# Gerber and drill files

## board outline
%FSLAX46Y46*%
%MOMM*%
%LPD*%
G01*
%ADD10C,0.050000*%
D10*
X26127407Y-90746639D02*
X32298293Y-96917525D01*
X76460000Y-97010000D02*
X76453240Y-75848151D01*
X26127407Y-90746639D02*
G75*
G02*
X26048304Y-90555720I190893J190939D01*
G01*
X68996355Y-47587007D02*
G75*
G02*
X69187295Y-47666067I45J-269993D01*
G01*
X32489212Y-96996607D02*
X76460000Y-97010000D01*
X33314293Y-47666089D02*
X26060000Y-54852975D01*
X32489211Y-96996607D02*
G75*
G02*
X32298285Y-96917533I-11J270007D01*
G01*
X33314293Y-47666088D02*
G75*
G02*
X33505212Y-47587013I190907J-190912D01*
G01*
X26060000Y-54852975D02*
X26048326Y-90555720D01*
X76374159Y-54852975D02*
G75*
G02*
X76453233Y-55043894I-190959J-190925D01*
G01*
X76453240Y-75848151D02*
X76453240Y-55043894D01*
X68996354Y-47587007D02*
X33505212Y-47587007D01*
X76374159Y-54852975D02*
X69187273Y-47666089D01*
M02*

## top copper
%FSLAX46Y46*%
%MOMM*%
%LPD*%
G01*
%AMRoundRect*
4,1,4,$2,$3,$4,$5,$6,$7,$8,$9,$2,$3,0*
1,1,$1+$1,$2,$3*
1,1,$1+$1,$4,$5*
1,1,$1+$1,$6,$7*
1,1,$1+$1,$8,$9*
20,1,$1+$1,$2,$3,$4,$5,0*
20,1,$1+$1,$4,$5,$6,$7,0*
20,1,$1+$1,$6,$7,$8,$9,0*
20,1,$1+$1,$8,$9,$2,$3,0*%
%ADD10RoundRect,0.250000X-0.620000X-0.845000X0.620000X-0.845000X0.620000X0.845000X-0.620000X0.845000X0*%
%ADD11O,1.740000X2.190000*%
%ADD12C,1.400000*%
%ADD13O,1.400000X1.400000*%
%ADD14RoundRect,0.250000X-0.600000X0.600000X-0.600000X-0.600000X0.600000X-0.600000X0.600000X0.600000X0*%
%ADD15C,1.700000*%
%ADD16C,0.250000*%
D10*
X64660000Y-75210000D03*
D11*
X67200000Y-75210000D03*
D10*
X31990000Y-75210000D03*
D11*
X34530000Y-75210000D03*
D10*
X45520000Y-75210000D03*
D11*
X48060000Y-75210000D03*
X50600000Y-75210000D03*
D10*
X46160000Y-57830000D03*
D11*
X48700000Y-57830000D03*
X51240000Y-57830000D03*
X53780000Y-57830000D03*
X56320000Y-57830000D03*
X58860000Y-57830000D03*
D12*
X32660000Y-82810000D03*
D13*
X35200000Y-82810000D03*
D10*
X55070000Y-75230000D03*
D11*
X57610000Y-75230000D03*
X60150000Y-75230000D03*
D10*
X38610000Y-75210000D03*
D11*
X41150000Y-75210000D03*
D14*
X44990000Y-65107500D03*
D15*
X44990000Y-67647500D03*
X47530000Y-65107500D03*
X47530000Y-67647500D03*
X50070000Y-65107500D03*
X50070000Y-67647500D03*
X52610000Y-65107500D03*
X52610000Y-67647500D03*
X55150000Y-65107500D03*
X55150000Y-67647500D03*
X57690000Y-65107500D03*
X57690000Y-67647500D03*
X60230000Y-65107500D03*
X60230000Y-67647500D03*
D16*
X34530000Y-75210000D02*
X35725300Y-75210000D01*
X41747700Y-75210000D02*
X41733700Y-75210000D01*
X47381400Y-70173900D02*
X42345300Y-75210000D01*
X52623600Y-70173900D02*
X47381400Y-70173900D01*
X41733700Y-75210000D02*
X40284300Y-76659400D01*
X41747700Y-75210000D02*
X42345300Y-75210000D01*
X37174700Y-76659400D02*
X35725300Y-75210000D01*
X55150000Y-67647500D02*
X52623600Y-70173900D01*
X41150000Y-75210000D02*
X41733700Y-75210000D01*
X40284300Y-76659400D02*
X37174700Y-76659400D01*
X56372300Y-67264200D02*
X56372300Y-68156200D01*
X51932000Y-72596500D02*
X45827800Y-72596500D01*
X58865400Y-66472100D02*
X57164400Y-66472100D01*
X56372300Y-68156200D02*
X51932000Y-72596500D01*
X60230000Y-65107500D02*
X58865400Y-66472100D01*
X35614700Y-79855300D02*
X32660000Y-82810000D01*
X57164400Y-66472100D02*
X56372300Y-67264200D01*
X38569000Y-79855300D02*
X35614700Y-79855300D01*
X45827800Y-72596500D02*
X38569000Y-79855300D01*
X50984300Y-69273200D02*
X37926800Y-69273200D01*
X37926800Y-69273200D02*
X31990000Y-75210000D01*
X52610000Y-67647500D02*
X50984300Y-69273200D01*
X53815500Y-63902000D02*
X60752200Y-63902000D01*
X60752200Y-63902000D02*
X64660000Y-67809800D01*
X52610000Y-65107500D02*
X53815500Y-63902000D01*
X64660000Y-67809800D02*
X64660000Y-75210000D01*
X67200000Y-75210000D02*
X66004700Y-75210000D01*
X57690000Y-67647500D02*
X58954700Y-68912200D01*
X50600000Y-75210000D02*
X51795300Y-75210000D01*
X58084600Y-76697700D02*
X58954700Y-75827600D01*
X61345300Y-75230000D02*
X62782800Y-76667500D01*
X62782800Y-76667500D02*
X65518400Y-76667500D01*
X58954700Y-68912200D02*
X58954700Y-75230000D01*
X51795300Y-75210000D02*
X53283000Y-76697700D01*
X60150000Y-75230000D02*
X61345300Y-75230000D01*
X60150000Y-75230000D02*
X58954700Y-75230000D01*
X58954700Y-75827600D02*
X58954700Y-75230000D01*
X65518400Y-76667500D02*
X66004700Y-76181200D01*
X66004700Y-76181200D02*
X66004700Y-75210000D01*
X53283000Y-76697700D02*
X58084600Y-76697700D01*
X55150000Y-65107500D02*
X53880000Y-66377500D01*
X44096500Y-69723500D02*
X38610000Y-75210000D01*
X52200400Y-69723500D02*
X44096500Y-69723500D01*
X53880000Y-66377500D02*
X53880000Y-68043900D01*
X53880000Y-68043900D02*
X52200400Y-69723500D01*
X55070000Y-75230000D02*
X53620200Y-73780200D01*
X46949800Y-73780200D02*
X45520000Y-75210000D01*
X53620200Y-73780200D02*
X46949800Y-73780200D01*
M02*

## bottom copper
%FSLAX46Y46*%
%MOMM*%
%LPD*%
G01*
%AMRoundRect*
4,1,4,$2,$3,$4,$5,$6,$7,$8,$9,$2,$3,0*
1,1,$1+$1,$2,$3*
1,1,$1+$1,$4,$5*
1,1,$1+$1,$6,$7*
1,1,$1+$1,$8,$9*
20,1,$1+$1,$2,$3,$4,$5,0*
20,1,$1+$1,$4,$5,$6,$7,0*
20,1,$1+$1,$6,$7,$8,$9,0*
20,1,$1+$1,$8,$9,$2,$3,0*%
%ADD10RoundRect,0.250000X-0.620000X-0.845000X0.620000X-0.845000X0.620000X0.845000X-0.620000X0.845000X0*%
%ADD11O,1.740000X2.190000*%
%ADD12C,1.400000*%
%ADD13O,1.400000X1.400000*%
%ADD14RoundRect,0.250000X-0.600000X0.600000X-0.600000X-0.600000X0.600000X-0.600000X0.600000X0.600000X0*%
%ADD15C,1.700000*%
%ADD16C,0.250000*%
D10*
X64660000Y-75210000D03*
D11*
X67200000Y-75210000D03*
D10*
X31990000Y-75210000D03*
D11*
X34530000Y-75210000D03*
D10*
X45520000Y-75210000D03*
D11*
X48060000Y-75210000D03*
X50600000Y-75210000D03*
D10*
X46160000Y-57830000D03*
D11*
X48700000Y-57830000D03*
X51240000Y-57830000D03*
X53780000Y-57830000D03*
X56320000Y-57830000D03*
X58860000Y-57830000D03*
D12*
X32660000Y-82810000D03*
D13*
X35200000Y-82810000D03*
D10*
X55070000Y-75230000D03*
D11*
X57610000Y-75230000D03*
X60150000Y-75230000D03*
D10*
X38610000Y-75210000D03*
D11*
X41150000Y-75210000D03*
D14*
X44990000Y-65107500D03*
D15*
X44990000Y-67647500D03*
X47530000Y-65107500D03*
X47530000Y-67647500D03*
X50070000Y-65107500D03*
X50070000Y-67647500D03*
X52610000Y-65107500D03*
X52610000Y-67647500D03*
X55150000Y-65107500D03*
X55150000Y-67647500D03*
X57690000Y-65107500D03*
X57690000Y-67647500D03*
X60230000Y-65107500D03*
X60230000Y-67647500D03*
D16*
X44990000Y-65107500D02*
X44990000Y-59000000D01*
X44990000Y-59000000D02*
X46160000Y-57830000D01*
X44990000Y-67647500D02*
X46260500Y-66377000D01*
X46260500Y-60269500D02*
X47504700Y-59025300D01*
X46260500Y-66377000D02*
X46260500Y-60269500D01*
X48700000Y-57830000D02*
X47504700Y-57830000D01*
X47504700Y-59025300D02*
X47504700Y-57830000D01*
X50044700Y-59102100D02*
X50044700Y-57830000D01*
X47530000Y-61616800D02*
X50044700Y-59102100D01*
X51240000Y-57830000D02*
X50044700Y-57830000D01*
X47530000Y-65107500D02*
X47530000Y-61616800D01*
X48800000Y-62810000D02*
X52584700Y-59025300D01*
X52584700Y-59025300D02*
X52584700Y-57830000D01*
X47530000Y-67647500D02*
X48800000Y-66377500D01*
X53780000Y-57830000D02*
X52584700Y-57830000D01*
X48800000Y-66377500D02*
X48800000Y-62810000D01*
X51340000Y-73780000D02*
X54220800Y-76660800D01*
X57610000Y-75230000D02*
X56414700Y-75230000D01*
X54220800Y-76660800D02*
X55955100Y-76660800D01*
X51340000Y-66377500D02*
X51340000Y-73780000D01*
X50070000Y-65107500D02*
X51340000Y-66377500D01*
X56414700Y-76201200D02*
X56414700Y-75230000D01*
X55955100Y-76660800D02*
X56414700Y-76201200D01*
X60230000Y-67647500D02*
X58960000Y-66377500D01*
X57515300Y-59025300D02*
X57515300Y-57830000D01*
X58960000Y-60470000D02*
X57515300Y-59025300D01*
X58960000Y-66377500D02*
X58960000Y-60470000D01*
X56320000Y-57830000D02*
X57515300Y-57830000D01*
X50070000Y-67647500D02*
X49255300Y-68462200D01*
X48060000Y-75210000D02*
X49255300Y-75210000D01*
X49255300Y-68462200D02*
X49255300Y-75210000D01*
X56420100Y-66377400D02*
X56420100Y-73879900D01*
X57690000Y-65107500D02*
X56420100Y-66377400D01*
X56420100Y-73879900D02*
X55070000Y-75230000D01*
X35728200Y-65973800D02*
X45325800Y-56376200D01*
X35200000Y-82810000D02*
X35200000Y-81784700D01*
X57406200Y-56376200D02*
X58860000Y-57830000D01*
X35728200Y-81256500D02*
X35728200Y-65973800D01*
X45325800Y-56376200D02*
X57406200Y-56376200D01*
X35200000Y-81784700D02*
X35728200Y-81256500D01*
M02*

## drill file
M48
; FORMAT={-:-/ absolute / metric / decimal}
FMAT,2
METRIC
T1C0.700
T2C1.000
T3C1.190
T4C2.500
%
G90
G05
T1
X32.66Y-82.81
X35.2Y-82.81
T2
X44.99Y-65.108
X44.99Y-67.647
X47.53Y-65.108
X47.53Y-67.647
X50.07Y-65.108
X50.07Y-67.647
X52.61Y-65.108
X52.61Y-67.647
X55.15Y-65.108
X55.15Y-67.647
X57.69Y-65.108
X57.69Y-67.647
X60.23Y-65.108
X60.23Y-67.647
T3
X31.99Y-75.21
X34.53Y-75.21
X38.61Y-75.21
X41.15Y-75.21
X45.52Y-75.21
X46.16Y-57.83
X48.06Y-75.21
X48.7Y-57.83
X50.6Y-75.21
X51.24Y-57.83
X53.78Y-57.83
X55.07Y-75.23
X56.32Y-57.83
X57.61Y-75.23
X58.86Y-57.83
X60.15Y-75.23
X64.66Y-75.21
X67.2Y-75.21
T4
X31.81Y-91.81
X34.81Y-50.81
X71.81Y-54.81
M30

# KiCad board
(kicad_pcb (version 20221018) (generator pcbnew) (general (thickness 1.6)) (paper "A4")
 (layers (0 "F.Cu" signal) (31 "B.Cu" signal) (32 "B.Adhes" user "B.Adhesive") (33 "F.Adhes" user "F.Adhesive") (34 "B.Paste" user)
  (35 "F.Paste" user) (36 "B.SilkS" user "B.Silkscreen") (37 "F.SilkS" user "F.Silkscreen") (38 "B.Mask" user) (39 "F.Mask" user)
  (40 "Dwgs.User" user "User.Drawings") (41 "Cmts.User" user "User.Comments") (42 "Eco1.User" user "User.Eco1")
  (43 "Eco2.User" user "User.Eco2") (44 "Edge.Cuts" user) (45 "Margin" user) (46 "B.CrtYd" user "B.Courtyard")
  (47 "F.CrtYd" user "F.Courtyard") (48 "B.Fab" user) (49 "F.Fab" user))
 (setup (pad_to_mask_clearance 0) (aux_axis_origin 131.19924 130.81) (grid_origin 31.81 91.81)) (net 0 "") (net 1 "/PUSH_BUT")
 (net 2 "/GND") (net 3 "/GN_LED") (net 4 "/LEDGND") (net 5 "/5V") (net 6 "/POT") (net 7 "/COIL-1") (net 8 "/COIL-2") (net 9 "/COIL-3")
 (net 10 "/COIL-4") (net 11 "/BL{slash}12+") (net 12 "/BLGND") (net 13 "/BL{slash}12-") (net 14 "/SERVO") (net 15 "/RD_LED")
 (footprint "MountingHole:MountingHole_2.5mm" (layer "F.Cu") (at 34.81 50.81)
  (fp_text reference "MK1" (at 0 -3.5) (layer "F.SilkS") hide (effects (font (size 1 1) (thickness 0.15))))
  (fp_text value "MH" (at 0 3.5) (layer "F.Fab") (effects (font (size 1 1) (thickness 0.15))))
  (pad "" np_thru_hole circle (at 0 0) (size 2.5 2.5) (drill 2.5) (layers "*.Cu" "*.Mask")))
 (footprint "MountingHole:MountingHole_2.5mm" (layer "F.Cu") (at 31.81 91.81)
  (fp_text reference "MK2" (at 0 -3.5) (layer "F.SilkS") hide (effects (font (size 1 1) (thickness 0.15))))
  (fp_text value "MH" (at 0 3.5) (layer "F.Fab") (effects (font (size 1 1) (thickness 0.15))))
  (pad "" np_thru_hole circle (at 0 0) (size 2.5 2.5) (drill 2.5) (layers "*.Cu" "*.Mask")))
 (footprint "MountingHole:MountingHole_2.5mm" (layer "F.Cu") (at 71.81 54.81)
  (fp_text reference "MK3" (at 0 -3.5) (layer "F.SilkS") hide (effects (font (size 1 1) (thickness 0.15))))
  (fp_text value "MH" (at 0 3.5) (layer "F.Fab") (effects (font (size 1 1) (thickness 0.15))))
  (pad "" np_thru_hole circle (at 0 0) (size 2.5 2.5) (drill 2.5) (layers "*.Cu" "*.Mask")))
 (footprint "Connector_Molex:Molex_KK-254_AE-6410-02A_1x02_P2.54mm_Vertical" (layer "F.Cu") (at 64.66 75.21)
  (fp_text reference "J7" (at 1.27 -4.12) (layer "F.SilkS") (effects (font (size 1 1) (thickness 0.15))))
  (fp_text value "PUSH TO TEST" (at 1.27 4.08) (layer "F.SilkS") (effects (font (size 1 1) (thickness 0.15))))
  (pad "1" thru_hole roundrect (at 0 0) (size 1.74 2.19) (drill 1.19) (layers "*.Cu" "*.Mask") (roundrect_rratio 0.1436781609)
   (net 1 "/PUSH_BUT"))
  (pad "2" thru_hole oval (at 2.54 0) (size 1.74 2.19) (drill 1.19) (layers "*.Cu" "*.Mask") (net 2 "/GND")))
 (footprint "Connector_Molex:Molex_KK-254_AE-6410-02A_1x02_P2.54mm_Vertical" (layer "F.Cu") (at 31.99 75.21)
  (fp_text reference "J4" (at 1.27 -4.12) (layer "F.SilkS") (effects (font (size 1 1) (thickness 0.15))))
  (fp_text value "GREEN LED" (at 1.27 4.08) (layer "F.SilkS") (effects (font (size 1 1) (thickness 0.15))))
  (pad "1" thru_hole roundrect (at 0 0) (size 1.74 2.19) (drill 1.19) (layers "*.Cu" "*.Mask") (roundrect_rratio 0.1436781609)
   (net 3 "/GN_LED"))
  (pad "2" thru_hole oval (at 2.54 0) (size 1.74 2.19) (drill 1.19) (layers "*.Cu" "*.Mask") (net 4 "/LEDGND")))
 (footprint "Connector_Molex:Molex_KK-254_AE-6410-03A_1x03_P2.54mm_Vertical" (layer "F.Cu") (at 45.52 75.21)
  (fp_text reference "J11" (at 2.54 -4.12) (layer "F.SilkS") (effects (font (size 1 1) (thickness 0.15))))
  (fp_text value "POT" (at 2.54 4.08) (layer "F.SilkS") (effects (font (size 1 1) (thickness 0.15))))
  (pad "1" thru_hole roundrect (at 0 0) (size 1.74 2.19) (drill 1.19) (layers "*.Cu" "*.Mask") (roundrect_rratio 0.1436781609) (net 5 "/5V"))
  (pad "2" thru_hole oval (at 2.54 0) (size 1.74 2.19) (drill 1.19) (layers "*.Cu" "*.Mask") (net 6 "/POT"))
  (pad "3" thru_hole oval (at 5.08 0) (size 1.74 2.19) (drill 1.19) (layers "*.Cu" "*.Mask") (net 2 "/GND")))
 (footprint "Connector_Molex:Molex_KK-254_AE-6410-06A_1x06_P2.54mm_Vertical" (layer "F.Cu") (at 46.16 57.83)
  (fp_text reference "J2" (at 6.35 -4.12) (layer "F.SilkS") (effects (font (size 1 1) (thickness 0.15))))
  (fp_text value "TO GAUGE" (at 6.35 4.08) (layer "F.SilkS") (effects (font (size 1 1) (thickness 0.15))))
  (pad "1" thru_hole roundrect (at 0 0) (size 1.74 2.19) (drill 1.19) (layers "*.Cu" "*.Mask") (roundrect_rratio 0.1436781609)
   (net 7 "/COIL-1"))
  (pad "2" thru_hole oval (at 2.54 0) (size 1.74 2.19) (drill 1.19) (layers "*.Cu" "*.Mask") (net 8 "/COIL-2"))
  (pad "3" thru_hole oval (at 5.08 0) (size 1.74 2.19) (drill 1.19) (layers "*.Cu" "*.Mask") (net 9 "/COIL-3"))
  (pad "4" thru_hole oval (at 7.62 0) (size 1.74 2.19) (drill 1.19) (layers "*.Cu" "*.Mask") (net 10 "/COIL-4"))
  (pad "5" thru_hole oval (at 10.16 0) (size 1.74 2.19) (drill 1.19) (layers "*.Cu" "*.Mask") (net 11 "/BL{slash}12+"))
  (pad "6" thru_hole oval (at 12.7 0) (size 1.74 2.19) (drill 1.19) (layers "*.Cu" "*.Mask") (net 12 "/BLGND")))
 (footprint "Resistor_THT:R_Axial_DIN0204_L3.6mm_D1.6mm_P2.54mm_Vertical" (layer "F.Cu") (at 32.66 82.81)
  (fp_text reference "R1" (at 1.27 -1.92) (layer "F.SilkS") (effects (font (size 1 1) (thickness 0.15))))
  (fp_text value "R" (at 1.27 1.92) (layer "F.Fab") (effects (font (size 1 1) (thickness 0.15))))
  (pad "1" thru_hole circle (at 0 0) (size 1.4 1.4) (drill 0.7) (layers "*.Cu" "*.Mask") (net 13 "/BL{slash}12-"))
  (pad "2" thru_hole oval (at 2.54 0) (size 1.4 1.4) (drill 0.7) (layers "*.Cu" "*.Mask") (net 12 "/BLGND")))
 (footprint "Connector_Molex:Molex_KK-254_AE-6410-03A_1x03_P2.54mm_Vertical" (layer "F.Cu") (at 55.07 75.23)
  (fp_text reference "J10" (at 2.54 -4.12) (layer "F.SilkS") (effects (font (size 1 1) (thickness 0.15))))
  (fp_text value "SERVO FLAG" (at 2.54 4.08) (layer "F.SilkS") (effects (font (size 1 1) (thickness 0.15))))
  (pad "1" thru_hole roundrect (at 0 0) (size 1.74 2.19) (drill 1.19) (layers "*.Cu" "*.Mask") (roundrect_rratio 0.1436781609) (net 5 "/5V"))
  (pad "2" thru_hole oval (at 2.54 0) (size 1.74 2.19) (drill 1.19) (layers "*.Cu" "*.Mask") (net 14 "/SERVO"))
  (pad "3" thru_hole oval (at 5.08 0) (size 1.74 2.19) (drill 1.19) (layers "*.Cu" "*.Mask") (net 2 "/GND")))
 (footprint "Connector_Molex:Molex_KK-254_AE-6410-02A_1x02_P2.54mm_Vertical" (layer "F.Cu") (at 38.61 75.21)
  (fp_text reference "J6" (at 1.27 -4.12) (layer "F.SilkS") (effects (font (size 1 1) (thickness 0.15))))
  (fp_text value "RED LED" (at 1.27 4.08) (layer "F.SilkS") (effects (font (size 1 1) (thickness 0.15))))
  (pad "1" thru_hole roundrect (at 0 0) (size 1.74 2.19) (drill 1.19) (layers "*.Cu" "*.Mask") (roundrect_rratio 0.1436781609)
   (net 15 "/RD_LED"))
  (pad "2" thru_hole oval (at 2.54 0) (size 1.74 2.19) (drill 1.19) (layers "*.Cu" "*.Mask") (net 4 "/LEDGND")))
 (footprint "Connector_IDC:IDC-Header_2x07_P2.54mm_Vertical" (layer "B.Cu") (at 44.99 65.1075 -90)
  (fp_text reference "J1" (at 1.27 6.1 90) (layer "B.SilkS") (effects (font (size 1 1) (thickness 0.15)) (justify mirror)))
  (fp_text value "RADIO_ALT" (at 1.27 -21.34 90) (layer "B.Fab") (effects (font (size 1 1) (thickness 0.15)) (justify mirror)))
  (pad "1" thru_hole roundrect (at 0 0 270) (size 1.7 1.7) (drill 1) (layers "*.Cu" "*.Mask") (roundrect_rratio 0.1470588235)
   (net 7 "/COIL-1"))
  (pad "2" thru_hole circle (at 2.54 0 270) (size 1.7 1.7) (drill 1) (layers "*.Cu" "*.Mask") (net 8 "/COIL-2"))
  (pad "3" thru_hole circle (at 0 -2.54 270) (size 1.7 1.7) (drill 1) (layers "*.Cu" "*.Mask") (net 9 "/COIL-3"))
  (pad "4" thru_hole circle (at 2.54 -2.54 270) (size 1.7 1.7) (drill 1) (layers "*.Cu" "*.Mask") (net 10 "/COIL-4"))
  (pad "5" thru_hole circle (at 0 -5.08 270) (size 1.7 1.7) (drill 1) (layers "*.Cu" "*.Mask") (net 14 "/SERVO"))
  (pad "6" thru_hole circle (at 2.54 -5.08 270) (size 1.7 1.7) (drill 1) (layers "*.Cu" "*.Mask") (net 6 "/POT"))
  (pad "7" thru_hole circle (at 0 -7.62 270) (size 1.7 1.7) (drill 1) (layers "*.Cu" "*.Mask") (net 1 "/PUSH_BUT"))
  (pad "8" thru_hole circle (at 2.54 -7.62 270) (size 1.7 1.7) (drill 1) (layers "*.Cu" "*.Mask") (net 3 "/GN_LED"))
  (pad "9" thru_hole circle (at 0 -10.16 270) (size 1.7 1.7) (drill 1) (layers "*.Cu" "*.Mask") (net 15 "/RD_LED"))
  (pad "10" thru_hole circle (at 2.54 -10.16 270) (size 1.7 1.7) (drill 1) (layers "*.Cu" "*.Mask") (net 4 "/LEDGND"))
  (pad "11" thru_hole circle (at 0 -12.7 270) (size 1.7 1.7) (drill 1) (layers "*.Cu" "*.Mask") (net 5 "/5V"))
  (pad "12" thru_hole circle (at 2.54 -12.7 270) (size 1.7 1.7) (drill 1) (layers "*.Cu" "*.Mask") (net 2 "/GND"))
  (pad "13" thru_hole circle (at 0 -15.24 270) (size 1.7 1.7) (drill 1) (layers "*.Cu" "*.Mask") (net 13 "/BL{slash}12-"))
  (pad "14" thru_hole circle (at 2.54 -15.24 270) (size 1.7 1.7) (drill 1) (layers "*.Cu" "*.Mask") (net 11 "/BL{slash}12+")))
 (gr_line (start 26.127407 90.746639) (end 32.298293 96.917525) (stroke (width 0.05) (type solid)) (layer "Edge.Cuts"))
 (gr_line (start 76.46 97.01) (end 76.45324 75.848151) (stroke (width 0.05) (type solid)) (layer "Edge.Cuts"))
 (gr_arc (start 26.127407 90.746639) (mid 26.068878 90.659045) (end 26.048326 90.55572) (stroke (width 0.05) (type solid))
  (layer "Edge.Cuts"))
 (gr_arc (start 68.996355 47.587007) (mid 69.099679 47.60756) (end 69.187273 47.666089) (stroke (width 0.05) (type solid))
  (layer "Edge.Cuts"))
 (gr_line (start 32.489212 96.996607) (end 76.46 97.01) (stroke (width 0.05) (type solid)) (layer "Edge.Cuts"))
 (gr_line (start 33.314293 47.666089) (end 26.06 54.852975) (stroke (width 0.05) (type solid)) (layer "Edge.Cuts"))
 (gr_arc (start 32.489211 96.996607) (mid 32.385887 96.976054) (end 32.298293 96.917525) (stroke (width 0.05) (type solid))
  (layer "Edge.Cuts"))
 (gr_arc (start 33.314293 47.666088) (mid 33.401887 47.607559) (end 33.505212 47.587007) (stroke (width 0.05) (type solid))
  (layer "Edge.Cuts"))
 (gr_line (start 26.06 54.852975) (end 26.048326 90.55572) (stroke (width 0.05) (type solid)) (layer "Edge.Cuts"))
 (gr_arc (start 76.374159 54.852975) (mid 76.432688 54.940569) (end 76.45324 55.043894) (stroke (width 0.05) (type solid))
  (layer "Edge.Cuts"))
 (gr_line (start 76.45324 75.848151) (end 76.45324 55.043894) (stroke (width 0.05) (type solid)) (layer "Edge.Cuts"))
 (gr_line (start 68.996354 47.587007) (end 33.505212 47.587007) (stroke (width 0.05) (type solid)) (layer "Edge.Cuts"))
 (gr_line (start 76.374159 54.852975) (end 69.187273 47.666089) (stroke (width 0.05) (type solid)) (layer "Edge.Cuts"))
 (segment (start 34.53 75.21) (end 35.7253 75.21) (width 0.25) (layer "F.Cu") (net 4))
 (segment (start 41.7477 75.21) (end 41.7337 75.21) (width 0.25) (layer "F.Cu") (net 4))
 (segment (start 47.3814 70.1739) (end 42.3453 75.21) (width 0.25) (layer "F.Cu") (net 4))
 (segment (start 52.6236 70.1739) (end 47.3814 70.1739) (width 0.25) (layer "F.Cu") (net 4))
 (segment (start 41.7337 75.21) (end 40.2843 76.6594) (width 0.25) (layer "F.Cu") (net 4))
 (segment (start 41.7477 75.21) (end 42.3453 75.21) (width 0.25) (layer "F.Cu") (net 4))
 (segment (start 37.1747 76.6594) (end 35.7253 75.21) (width 0.25) (layer "F.Cu") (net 4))
 (segment (start 55.15 67.6475) (end 52.6236 70.1739) (width 0.25) (layer "F.Cu") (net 4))
 (segment (start 41.15 75.21) (end 41.7337 75.21) (width 0.25) (layer "F.Cu") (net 4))
 (segment (start 40.2843 76.6594) (end 37.1747 76.6594) (width 0.25) (layer "F.Cu") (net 4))
 (segment (start 44.99 65.1075) (end 44.99 59) (width 0.25) (layer "B.Cu") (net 7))
 (segment (start 44.99 59) (end 46.16 57.83) (width 0.25) (layer "B.Cu") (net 7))
 (segment (start 44.99 67.6475) (end 46.2605 66.377) (width 0.25) (layer "B.Cu") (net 8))
 (segment (start 46.2605 60.2695) (end 47.5047 59.0253) (width 0.25) (layer "B.Cu") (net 8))
 (segment (start 46.2605 66.377) (end 46.2605 60.2695) (width 0.25) (layer "B.Cu") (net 8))
 (segment (start 48.7 57.83) (end 47.5047 57.83) (width 0.25) (layer "B.Cu") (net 8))
 (segment (start 47.5047 59.0253) (end 47.5047 57.83) (width 0.25) (layer "B.Cu") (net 8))
 (segment (start 50.0447 59.1021) (end 50.0447 57.83) (width 0.25) (layer "B.Cu") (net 9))
 (segment (start 47.53 61.6168) (end 50.0447 59.1021) (width 0.25) (layer "B.Cu") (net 9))
 (segment (start 51.24 57.83) (end 50.0447 57.83) (width 0.25) (layer "B.Cu") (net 9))
 (segment (start 47.53 65.1075) (end 47.53 61.6168) (width 0.25) (layer "B.Cu") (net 9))
 (segment (start 48.8 62.81) (end 52.5847 59.0253) (width 0.25) (layer "B.Cu") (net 10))
 (segment (start 52.5847 59.0253) (end 52.5847 57.83) (width 0.25) (layer "B.Cu") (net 10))
 (segment (start 47.53 67.6475) (end 48.8 66.3775) (width 0.25) (layer "B.Cu") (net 10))
 (segment (start 53.78 57.83) (end 52.5847 57.83) (width 0.25) (layer "B.Cu") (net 10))
 (segment (start 48.8 66.3775) (end 48.8 62.81) (width 0.25) (layer "B.Cu") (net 10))
 (segment (start 51.34 73.78) (end 54.2208 76.6608) (width 0.25) (layer "B.Cu") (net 14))
 (segment (start 57.61 75.23) (end 56.4147 75.23) (width 0.25) (layer "B.Cu") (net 14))
 (segment (start 54.2208 76.6608) (end 55.9551 76.6608) (width 0.25) (layer "B.Cu") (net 14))
 (segment (start 51.34 66.3775) (end 51.34 73.78) (width 0.25) (layer "B.Cu") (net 14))
 (segment (start 50.07 65.1075) (end 51.34 66.3775) (width 0.25) (layer "B.Cu") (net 14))
 (segment (start 56.4147 76.2012) (end 56.4147 75.23) (width 0.25) (layer "B.Cu") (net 14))
 (segment (start 55.9551 76.6608) (end 56.4147 76.2012) (width 0.25) (layer "B.Cu") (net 14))
 (segment (start 60.23 67.6475) (end 58.96 66.3775) (width 0.25) (layer "B.Cu") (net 11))
 (segment (start 57.5153 59.0253) (end 57.5153 57.83) (width 0.25) (layer "B.Cu") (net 11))
 (segment (start 58.96 60.47) (end 57.5153 59.0253) (width 0.25) (layer "B.Cu") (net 11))
 (segment (start 58.96 66.3775) (end 58.96 60.47) (width 0.25) (layer "B.Cu") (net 11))
 (segment (start 56.32 57.83) (end 57.5153 57.83) (width 0.25) (layer "B.Cu") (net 11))
 (segment (start 56.3723 67.2642) (end 56.3723 68.1562) (width 0.25) (layer "F.Cu") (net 13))
 (segment (start 51.932 72.5965) (end 45.8278 72.5965) (width 0.25) (layer "F.Cu") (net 13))
 (segment (start 58.8654 66.4721) (end 57.1644 66.4721) (width 0.25) (layer "F.Cu") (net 13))
 (segment (start 56.3723 68.1562) (end 51.932 72.5965) (width 0.25) (layer "F.Cu") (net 13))
 (segment (start 60.23 65.1075) (end 58.8654 66.4721) (width 0.25) (layer "F.Cu") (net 13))
 (segment (start 35.6147 79.8553) (end 32.66 82.81) (width 0.25) (layer "F.Cu") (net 13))
 (segment (start 57.1644 66.4721) (end 56.3723 67.2642) (width 0.25) (layer "F.Cu") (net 13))
 (segment (start 38.569 79.8553) (end 35.6147 79.8553) (width 0.25) (layer "F.Cu") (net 13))
 (segment (start 45.8278 72.5965) (end 38.569 79.8553) (width 0.25) (layer "F.Cu") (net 13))
 (segment (start 50.9843 69.2732) (end 37.9268 69.2732) (width 0.25) (layer "F.Cu") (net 3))
 (segment (start 37.9268 69.2732) (end 31.99 75.21) (width 0.25) (layer "F.Cu") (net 3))
 (segment (start 52.61 67.6475) (end 50.9843 69.2732) (width 0.25) (layer "F.Cu") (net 3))
 (segment (start 50.07 67.6475) (end 49.2553 68.4622) (width 0.25) (layer "B.Cu") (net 6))
 (segment (start 48.06 75.21) (end 49.2553 75.21) (width 0.25) (layer "B.Cu") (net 6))
 (segment (start 49.2553 68.4622) (end 49.2553 75.21) (width 0.25) (layer "B.Cu") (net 6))
 (segment (start 53.8155 63.902) (end 60.7522 63.902) (width 0.25) (layer "F.Cu") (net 1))
 (segment (start 60.7522 63.902) (end 64.66 67.8098) (width 0.25) (layer "F.Cu") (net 1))
 (segment (start 52.61 65.1075) (end 53.8155 63.902) (width 0.25) (layer "F.Cu") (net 1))
 (segment (start 64.66 67.8098) (end 64.66 75.21) (width 0.25) (layer "F.Cu") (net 1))
 (segment (start 67.2 75.21) (end 66.0047 75.21) (width 0.25) (layer "F.Cu") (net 2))
 (segment (start 57.69 67.6475) (end 58.9547 68.9122) (width 0.25) (layer "F.Cu") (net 2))
 (segment (start 50.6 75.21) (end 51.7953 75.21) (width 0.25) (layer "F.Cu") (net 2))
 (segment (start 58.0846 76.6977) (end 58.9547 75.8276) (width 0.25) (layer "F.Cu") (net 2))
 (segment (start 61.3453 75.23) (end 62.7828 76.6675) (width 0.25) (layer "F.Cu") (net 2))
 (segment (start 62.7828 76.6675) (end 65.5184 76.6675) (width 0.25) (layer "F.Cu") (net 2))
 (segment (start 58.9547 68.9122) (end 58.9547 75.23) (width 0.25) (layer "F.Cu") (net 2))
 (segment (start 51.7953 75.21) (end 53.283 76.6977) (width 0.25) (layer "F.Cu") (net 2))
 (segment (start 60.15 75.23) (end 61.3453 75.23) (width 0.25) (layer "F.Cu") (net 2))
 (segment (start 60.15 75.23) (end 58.9547 75.23) (width 0.25) (layer "F.Cu") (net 2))
 (segment (start 58.9547 75.8276) (end 58.9547 75.23) (width 0.25) (layer "F.Cu") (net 2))
 (segment (start 65.5184 76.6675) (end 66.0047 76.1812) (width 0.25) (layer "F.Cu") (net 2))
 (segment (start 66.0047 76.1812) (end 66.0047 75.21) (width 0.25) (layer "F.Cu") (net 2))
 (segment (start 53.283 76.6977) (end 58.0846 76.6977) (width 0.25) (layer "F.Cu") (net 2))
 (segment (start 55.15 65.1075) (end 53.88 66.3775) (width 0.25) (layer "F.Cu") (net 15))
 (segment (start 44.0965 69.7235) (end 38.61 75.21) (width 0.25) (layer "F.Cu") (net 15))
 (segment (start 52.2004 69.7235) (end 44.0965 69.7235) (width 0.25) (layer "F.Cu") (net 15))
 (segment (start 53.88 66.3775) (end 53.88 68.0439) (width 0.25) (layer "F.Cu") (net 15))
 (segment (start 53.88 68.0439) (end 52.2004 69.7235) (width 0.25) (layer "F.Cu") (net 15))
 (segment (start 55.07 75.23) (end 53.6202 73.7802) (width 0.25) (layer "F.Cu") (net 5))
 (segment (start 46.9498 73.7802) (end 45.52 75.21) (width 0.25) (layer "F.Cu") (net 5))
 (segment (start 53.6202 73.7802) (end 46.9498 73.7802) (width 0.25) (layer "F.Cu") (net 5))
 (segment (start 56.4201 66.3774) (end 56.4201 73.8799) (width 0.25) (layer "B.Cu") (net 5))
 (segment (start 57.69 65.1075) (end 56.4201 66.3774) (width 0.25) (layer "B.Cu") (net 5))
 (segment (start 56.4201 73.8799) (end 55.07 75.23) (width 0.25) (layer "B.Cu") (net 5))
 (segment (start 35.7282 65.9738) (end 45.3258 56.3762) (width 0.25) (layer "B.Cu") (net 12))
 (segment (start 35.2 82.81) (end 35.2 81.7847) (width 0.25) (layer "B.Cu") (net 12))
 (segment (start 57.4062 56.3762) (end 58.86 57.83) (width 0.25) (layer "B.Cu") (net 12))
 (segment (start 35.7282 81.2565) (end 35.7282 65.9738) (width 0.25) (layer "B.Cu") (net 12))
 (segment (start 45.3258 56.3762) (end 57.4062 56.3762) (width 0.25) (layer "B.Cu") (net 12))
 (segment (start 35.2 81.7847) (end 35.7282 81.2565) (width 0.25) (layer "B.Cu") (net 12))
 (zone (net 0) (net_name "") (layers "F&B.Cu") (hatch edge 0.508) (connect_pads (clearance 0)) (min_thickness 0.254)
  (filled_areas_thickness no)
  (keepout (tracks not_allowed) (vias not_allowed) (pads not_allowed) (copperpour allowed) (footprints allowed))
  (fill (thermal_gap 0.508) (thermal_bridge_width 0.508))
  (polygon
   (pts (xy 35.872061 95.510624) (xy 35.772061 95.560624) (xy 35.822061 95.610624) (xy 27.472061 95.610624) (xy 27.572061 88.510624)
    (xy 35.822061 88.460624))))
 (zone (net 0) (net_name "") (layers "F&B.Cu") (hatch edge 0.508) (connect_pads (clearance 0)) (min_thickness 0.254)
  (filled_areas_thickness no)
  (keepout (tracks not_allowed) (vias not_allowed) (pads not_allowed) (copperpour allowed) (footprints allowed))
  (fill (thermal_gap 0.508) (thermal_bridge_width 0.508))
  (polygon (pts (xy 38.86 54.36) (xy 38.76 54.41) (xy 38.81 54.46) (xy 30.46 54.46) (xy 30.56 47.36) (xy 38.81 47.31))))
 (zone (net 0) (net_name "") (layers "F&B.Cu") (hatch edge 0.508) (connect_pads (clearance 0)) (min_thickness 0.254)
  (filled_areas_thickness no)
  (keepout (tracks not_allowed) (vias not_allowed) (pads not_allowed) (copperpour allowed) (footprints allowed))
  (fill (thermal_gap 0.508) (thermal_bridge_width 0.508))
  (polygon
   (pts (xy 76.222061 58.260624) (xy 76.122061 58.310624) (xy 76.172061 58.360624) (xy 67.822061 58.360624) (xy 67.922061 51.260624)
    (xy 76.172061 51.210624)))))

